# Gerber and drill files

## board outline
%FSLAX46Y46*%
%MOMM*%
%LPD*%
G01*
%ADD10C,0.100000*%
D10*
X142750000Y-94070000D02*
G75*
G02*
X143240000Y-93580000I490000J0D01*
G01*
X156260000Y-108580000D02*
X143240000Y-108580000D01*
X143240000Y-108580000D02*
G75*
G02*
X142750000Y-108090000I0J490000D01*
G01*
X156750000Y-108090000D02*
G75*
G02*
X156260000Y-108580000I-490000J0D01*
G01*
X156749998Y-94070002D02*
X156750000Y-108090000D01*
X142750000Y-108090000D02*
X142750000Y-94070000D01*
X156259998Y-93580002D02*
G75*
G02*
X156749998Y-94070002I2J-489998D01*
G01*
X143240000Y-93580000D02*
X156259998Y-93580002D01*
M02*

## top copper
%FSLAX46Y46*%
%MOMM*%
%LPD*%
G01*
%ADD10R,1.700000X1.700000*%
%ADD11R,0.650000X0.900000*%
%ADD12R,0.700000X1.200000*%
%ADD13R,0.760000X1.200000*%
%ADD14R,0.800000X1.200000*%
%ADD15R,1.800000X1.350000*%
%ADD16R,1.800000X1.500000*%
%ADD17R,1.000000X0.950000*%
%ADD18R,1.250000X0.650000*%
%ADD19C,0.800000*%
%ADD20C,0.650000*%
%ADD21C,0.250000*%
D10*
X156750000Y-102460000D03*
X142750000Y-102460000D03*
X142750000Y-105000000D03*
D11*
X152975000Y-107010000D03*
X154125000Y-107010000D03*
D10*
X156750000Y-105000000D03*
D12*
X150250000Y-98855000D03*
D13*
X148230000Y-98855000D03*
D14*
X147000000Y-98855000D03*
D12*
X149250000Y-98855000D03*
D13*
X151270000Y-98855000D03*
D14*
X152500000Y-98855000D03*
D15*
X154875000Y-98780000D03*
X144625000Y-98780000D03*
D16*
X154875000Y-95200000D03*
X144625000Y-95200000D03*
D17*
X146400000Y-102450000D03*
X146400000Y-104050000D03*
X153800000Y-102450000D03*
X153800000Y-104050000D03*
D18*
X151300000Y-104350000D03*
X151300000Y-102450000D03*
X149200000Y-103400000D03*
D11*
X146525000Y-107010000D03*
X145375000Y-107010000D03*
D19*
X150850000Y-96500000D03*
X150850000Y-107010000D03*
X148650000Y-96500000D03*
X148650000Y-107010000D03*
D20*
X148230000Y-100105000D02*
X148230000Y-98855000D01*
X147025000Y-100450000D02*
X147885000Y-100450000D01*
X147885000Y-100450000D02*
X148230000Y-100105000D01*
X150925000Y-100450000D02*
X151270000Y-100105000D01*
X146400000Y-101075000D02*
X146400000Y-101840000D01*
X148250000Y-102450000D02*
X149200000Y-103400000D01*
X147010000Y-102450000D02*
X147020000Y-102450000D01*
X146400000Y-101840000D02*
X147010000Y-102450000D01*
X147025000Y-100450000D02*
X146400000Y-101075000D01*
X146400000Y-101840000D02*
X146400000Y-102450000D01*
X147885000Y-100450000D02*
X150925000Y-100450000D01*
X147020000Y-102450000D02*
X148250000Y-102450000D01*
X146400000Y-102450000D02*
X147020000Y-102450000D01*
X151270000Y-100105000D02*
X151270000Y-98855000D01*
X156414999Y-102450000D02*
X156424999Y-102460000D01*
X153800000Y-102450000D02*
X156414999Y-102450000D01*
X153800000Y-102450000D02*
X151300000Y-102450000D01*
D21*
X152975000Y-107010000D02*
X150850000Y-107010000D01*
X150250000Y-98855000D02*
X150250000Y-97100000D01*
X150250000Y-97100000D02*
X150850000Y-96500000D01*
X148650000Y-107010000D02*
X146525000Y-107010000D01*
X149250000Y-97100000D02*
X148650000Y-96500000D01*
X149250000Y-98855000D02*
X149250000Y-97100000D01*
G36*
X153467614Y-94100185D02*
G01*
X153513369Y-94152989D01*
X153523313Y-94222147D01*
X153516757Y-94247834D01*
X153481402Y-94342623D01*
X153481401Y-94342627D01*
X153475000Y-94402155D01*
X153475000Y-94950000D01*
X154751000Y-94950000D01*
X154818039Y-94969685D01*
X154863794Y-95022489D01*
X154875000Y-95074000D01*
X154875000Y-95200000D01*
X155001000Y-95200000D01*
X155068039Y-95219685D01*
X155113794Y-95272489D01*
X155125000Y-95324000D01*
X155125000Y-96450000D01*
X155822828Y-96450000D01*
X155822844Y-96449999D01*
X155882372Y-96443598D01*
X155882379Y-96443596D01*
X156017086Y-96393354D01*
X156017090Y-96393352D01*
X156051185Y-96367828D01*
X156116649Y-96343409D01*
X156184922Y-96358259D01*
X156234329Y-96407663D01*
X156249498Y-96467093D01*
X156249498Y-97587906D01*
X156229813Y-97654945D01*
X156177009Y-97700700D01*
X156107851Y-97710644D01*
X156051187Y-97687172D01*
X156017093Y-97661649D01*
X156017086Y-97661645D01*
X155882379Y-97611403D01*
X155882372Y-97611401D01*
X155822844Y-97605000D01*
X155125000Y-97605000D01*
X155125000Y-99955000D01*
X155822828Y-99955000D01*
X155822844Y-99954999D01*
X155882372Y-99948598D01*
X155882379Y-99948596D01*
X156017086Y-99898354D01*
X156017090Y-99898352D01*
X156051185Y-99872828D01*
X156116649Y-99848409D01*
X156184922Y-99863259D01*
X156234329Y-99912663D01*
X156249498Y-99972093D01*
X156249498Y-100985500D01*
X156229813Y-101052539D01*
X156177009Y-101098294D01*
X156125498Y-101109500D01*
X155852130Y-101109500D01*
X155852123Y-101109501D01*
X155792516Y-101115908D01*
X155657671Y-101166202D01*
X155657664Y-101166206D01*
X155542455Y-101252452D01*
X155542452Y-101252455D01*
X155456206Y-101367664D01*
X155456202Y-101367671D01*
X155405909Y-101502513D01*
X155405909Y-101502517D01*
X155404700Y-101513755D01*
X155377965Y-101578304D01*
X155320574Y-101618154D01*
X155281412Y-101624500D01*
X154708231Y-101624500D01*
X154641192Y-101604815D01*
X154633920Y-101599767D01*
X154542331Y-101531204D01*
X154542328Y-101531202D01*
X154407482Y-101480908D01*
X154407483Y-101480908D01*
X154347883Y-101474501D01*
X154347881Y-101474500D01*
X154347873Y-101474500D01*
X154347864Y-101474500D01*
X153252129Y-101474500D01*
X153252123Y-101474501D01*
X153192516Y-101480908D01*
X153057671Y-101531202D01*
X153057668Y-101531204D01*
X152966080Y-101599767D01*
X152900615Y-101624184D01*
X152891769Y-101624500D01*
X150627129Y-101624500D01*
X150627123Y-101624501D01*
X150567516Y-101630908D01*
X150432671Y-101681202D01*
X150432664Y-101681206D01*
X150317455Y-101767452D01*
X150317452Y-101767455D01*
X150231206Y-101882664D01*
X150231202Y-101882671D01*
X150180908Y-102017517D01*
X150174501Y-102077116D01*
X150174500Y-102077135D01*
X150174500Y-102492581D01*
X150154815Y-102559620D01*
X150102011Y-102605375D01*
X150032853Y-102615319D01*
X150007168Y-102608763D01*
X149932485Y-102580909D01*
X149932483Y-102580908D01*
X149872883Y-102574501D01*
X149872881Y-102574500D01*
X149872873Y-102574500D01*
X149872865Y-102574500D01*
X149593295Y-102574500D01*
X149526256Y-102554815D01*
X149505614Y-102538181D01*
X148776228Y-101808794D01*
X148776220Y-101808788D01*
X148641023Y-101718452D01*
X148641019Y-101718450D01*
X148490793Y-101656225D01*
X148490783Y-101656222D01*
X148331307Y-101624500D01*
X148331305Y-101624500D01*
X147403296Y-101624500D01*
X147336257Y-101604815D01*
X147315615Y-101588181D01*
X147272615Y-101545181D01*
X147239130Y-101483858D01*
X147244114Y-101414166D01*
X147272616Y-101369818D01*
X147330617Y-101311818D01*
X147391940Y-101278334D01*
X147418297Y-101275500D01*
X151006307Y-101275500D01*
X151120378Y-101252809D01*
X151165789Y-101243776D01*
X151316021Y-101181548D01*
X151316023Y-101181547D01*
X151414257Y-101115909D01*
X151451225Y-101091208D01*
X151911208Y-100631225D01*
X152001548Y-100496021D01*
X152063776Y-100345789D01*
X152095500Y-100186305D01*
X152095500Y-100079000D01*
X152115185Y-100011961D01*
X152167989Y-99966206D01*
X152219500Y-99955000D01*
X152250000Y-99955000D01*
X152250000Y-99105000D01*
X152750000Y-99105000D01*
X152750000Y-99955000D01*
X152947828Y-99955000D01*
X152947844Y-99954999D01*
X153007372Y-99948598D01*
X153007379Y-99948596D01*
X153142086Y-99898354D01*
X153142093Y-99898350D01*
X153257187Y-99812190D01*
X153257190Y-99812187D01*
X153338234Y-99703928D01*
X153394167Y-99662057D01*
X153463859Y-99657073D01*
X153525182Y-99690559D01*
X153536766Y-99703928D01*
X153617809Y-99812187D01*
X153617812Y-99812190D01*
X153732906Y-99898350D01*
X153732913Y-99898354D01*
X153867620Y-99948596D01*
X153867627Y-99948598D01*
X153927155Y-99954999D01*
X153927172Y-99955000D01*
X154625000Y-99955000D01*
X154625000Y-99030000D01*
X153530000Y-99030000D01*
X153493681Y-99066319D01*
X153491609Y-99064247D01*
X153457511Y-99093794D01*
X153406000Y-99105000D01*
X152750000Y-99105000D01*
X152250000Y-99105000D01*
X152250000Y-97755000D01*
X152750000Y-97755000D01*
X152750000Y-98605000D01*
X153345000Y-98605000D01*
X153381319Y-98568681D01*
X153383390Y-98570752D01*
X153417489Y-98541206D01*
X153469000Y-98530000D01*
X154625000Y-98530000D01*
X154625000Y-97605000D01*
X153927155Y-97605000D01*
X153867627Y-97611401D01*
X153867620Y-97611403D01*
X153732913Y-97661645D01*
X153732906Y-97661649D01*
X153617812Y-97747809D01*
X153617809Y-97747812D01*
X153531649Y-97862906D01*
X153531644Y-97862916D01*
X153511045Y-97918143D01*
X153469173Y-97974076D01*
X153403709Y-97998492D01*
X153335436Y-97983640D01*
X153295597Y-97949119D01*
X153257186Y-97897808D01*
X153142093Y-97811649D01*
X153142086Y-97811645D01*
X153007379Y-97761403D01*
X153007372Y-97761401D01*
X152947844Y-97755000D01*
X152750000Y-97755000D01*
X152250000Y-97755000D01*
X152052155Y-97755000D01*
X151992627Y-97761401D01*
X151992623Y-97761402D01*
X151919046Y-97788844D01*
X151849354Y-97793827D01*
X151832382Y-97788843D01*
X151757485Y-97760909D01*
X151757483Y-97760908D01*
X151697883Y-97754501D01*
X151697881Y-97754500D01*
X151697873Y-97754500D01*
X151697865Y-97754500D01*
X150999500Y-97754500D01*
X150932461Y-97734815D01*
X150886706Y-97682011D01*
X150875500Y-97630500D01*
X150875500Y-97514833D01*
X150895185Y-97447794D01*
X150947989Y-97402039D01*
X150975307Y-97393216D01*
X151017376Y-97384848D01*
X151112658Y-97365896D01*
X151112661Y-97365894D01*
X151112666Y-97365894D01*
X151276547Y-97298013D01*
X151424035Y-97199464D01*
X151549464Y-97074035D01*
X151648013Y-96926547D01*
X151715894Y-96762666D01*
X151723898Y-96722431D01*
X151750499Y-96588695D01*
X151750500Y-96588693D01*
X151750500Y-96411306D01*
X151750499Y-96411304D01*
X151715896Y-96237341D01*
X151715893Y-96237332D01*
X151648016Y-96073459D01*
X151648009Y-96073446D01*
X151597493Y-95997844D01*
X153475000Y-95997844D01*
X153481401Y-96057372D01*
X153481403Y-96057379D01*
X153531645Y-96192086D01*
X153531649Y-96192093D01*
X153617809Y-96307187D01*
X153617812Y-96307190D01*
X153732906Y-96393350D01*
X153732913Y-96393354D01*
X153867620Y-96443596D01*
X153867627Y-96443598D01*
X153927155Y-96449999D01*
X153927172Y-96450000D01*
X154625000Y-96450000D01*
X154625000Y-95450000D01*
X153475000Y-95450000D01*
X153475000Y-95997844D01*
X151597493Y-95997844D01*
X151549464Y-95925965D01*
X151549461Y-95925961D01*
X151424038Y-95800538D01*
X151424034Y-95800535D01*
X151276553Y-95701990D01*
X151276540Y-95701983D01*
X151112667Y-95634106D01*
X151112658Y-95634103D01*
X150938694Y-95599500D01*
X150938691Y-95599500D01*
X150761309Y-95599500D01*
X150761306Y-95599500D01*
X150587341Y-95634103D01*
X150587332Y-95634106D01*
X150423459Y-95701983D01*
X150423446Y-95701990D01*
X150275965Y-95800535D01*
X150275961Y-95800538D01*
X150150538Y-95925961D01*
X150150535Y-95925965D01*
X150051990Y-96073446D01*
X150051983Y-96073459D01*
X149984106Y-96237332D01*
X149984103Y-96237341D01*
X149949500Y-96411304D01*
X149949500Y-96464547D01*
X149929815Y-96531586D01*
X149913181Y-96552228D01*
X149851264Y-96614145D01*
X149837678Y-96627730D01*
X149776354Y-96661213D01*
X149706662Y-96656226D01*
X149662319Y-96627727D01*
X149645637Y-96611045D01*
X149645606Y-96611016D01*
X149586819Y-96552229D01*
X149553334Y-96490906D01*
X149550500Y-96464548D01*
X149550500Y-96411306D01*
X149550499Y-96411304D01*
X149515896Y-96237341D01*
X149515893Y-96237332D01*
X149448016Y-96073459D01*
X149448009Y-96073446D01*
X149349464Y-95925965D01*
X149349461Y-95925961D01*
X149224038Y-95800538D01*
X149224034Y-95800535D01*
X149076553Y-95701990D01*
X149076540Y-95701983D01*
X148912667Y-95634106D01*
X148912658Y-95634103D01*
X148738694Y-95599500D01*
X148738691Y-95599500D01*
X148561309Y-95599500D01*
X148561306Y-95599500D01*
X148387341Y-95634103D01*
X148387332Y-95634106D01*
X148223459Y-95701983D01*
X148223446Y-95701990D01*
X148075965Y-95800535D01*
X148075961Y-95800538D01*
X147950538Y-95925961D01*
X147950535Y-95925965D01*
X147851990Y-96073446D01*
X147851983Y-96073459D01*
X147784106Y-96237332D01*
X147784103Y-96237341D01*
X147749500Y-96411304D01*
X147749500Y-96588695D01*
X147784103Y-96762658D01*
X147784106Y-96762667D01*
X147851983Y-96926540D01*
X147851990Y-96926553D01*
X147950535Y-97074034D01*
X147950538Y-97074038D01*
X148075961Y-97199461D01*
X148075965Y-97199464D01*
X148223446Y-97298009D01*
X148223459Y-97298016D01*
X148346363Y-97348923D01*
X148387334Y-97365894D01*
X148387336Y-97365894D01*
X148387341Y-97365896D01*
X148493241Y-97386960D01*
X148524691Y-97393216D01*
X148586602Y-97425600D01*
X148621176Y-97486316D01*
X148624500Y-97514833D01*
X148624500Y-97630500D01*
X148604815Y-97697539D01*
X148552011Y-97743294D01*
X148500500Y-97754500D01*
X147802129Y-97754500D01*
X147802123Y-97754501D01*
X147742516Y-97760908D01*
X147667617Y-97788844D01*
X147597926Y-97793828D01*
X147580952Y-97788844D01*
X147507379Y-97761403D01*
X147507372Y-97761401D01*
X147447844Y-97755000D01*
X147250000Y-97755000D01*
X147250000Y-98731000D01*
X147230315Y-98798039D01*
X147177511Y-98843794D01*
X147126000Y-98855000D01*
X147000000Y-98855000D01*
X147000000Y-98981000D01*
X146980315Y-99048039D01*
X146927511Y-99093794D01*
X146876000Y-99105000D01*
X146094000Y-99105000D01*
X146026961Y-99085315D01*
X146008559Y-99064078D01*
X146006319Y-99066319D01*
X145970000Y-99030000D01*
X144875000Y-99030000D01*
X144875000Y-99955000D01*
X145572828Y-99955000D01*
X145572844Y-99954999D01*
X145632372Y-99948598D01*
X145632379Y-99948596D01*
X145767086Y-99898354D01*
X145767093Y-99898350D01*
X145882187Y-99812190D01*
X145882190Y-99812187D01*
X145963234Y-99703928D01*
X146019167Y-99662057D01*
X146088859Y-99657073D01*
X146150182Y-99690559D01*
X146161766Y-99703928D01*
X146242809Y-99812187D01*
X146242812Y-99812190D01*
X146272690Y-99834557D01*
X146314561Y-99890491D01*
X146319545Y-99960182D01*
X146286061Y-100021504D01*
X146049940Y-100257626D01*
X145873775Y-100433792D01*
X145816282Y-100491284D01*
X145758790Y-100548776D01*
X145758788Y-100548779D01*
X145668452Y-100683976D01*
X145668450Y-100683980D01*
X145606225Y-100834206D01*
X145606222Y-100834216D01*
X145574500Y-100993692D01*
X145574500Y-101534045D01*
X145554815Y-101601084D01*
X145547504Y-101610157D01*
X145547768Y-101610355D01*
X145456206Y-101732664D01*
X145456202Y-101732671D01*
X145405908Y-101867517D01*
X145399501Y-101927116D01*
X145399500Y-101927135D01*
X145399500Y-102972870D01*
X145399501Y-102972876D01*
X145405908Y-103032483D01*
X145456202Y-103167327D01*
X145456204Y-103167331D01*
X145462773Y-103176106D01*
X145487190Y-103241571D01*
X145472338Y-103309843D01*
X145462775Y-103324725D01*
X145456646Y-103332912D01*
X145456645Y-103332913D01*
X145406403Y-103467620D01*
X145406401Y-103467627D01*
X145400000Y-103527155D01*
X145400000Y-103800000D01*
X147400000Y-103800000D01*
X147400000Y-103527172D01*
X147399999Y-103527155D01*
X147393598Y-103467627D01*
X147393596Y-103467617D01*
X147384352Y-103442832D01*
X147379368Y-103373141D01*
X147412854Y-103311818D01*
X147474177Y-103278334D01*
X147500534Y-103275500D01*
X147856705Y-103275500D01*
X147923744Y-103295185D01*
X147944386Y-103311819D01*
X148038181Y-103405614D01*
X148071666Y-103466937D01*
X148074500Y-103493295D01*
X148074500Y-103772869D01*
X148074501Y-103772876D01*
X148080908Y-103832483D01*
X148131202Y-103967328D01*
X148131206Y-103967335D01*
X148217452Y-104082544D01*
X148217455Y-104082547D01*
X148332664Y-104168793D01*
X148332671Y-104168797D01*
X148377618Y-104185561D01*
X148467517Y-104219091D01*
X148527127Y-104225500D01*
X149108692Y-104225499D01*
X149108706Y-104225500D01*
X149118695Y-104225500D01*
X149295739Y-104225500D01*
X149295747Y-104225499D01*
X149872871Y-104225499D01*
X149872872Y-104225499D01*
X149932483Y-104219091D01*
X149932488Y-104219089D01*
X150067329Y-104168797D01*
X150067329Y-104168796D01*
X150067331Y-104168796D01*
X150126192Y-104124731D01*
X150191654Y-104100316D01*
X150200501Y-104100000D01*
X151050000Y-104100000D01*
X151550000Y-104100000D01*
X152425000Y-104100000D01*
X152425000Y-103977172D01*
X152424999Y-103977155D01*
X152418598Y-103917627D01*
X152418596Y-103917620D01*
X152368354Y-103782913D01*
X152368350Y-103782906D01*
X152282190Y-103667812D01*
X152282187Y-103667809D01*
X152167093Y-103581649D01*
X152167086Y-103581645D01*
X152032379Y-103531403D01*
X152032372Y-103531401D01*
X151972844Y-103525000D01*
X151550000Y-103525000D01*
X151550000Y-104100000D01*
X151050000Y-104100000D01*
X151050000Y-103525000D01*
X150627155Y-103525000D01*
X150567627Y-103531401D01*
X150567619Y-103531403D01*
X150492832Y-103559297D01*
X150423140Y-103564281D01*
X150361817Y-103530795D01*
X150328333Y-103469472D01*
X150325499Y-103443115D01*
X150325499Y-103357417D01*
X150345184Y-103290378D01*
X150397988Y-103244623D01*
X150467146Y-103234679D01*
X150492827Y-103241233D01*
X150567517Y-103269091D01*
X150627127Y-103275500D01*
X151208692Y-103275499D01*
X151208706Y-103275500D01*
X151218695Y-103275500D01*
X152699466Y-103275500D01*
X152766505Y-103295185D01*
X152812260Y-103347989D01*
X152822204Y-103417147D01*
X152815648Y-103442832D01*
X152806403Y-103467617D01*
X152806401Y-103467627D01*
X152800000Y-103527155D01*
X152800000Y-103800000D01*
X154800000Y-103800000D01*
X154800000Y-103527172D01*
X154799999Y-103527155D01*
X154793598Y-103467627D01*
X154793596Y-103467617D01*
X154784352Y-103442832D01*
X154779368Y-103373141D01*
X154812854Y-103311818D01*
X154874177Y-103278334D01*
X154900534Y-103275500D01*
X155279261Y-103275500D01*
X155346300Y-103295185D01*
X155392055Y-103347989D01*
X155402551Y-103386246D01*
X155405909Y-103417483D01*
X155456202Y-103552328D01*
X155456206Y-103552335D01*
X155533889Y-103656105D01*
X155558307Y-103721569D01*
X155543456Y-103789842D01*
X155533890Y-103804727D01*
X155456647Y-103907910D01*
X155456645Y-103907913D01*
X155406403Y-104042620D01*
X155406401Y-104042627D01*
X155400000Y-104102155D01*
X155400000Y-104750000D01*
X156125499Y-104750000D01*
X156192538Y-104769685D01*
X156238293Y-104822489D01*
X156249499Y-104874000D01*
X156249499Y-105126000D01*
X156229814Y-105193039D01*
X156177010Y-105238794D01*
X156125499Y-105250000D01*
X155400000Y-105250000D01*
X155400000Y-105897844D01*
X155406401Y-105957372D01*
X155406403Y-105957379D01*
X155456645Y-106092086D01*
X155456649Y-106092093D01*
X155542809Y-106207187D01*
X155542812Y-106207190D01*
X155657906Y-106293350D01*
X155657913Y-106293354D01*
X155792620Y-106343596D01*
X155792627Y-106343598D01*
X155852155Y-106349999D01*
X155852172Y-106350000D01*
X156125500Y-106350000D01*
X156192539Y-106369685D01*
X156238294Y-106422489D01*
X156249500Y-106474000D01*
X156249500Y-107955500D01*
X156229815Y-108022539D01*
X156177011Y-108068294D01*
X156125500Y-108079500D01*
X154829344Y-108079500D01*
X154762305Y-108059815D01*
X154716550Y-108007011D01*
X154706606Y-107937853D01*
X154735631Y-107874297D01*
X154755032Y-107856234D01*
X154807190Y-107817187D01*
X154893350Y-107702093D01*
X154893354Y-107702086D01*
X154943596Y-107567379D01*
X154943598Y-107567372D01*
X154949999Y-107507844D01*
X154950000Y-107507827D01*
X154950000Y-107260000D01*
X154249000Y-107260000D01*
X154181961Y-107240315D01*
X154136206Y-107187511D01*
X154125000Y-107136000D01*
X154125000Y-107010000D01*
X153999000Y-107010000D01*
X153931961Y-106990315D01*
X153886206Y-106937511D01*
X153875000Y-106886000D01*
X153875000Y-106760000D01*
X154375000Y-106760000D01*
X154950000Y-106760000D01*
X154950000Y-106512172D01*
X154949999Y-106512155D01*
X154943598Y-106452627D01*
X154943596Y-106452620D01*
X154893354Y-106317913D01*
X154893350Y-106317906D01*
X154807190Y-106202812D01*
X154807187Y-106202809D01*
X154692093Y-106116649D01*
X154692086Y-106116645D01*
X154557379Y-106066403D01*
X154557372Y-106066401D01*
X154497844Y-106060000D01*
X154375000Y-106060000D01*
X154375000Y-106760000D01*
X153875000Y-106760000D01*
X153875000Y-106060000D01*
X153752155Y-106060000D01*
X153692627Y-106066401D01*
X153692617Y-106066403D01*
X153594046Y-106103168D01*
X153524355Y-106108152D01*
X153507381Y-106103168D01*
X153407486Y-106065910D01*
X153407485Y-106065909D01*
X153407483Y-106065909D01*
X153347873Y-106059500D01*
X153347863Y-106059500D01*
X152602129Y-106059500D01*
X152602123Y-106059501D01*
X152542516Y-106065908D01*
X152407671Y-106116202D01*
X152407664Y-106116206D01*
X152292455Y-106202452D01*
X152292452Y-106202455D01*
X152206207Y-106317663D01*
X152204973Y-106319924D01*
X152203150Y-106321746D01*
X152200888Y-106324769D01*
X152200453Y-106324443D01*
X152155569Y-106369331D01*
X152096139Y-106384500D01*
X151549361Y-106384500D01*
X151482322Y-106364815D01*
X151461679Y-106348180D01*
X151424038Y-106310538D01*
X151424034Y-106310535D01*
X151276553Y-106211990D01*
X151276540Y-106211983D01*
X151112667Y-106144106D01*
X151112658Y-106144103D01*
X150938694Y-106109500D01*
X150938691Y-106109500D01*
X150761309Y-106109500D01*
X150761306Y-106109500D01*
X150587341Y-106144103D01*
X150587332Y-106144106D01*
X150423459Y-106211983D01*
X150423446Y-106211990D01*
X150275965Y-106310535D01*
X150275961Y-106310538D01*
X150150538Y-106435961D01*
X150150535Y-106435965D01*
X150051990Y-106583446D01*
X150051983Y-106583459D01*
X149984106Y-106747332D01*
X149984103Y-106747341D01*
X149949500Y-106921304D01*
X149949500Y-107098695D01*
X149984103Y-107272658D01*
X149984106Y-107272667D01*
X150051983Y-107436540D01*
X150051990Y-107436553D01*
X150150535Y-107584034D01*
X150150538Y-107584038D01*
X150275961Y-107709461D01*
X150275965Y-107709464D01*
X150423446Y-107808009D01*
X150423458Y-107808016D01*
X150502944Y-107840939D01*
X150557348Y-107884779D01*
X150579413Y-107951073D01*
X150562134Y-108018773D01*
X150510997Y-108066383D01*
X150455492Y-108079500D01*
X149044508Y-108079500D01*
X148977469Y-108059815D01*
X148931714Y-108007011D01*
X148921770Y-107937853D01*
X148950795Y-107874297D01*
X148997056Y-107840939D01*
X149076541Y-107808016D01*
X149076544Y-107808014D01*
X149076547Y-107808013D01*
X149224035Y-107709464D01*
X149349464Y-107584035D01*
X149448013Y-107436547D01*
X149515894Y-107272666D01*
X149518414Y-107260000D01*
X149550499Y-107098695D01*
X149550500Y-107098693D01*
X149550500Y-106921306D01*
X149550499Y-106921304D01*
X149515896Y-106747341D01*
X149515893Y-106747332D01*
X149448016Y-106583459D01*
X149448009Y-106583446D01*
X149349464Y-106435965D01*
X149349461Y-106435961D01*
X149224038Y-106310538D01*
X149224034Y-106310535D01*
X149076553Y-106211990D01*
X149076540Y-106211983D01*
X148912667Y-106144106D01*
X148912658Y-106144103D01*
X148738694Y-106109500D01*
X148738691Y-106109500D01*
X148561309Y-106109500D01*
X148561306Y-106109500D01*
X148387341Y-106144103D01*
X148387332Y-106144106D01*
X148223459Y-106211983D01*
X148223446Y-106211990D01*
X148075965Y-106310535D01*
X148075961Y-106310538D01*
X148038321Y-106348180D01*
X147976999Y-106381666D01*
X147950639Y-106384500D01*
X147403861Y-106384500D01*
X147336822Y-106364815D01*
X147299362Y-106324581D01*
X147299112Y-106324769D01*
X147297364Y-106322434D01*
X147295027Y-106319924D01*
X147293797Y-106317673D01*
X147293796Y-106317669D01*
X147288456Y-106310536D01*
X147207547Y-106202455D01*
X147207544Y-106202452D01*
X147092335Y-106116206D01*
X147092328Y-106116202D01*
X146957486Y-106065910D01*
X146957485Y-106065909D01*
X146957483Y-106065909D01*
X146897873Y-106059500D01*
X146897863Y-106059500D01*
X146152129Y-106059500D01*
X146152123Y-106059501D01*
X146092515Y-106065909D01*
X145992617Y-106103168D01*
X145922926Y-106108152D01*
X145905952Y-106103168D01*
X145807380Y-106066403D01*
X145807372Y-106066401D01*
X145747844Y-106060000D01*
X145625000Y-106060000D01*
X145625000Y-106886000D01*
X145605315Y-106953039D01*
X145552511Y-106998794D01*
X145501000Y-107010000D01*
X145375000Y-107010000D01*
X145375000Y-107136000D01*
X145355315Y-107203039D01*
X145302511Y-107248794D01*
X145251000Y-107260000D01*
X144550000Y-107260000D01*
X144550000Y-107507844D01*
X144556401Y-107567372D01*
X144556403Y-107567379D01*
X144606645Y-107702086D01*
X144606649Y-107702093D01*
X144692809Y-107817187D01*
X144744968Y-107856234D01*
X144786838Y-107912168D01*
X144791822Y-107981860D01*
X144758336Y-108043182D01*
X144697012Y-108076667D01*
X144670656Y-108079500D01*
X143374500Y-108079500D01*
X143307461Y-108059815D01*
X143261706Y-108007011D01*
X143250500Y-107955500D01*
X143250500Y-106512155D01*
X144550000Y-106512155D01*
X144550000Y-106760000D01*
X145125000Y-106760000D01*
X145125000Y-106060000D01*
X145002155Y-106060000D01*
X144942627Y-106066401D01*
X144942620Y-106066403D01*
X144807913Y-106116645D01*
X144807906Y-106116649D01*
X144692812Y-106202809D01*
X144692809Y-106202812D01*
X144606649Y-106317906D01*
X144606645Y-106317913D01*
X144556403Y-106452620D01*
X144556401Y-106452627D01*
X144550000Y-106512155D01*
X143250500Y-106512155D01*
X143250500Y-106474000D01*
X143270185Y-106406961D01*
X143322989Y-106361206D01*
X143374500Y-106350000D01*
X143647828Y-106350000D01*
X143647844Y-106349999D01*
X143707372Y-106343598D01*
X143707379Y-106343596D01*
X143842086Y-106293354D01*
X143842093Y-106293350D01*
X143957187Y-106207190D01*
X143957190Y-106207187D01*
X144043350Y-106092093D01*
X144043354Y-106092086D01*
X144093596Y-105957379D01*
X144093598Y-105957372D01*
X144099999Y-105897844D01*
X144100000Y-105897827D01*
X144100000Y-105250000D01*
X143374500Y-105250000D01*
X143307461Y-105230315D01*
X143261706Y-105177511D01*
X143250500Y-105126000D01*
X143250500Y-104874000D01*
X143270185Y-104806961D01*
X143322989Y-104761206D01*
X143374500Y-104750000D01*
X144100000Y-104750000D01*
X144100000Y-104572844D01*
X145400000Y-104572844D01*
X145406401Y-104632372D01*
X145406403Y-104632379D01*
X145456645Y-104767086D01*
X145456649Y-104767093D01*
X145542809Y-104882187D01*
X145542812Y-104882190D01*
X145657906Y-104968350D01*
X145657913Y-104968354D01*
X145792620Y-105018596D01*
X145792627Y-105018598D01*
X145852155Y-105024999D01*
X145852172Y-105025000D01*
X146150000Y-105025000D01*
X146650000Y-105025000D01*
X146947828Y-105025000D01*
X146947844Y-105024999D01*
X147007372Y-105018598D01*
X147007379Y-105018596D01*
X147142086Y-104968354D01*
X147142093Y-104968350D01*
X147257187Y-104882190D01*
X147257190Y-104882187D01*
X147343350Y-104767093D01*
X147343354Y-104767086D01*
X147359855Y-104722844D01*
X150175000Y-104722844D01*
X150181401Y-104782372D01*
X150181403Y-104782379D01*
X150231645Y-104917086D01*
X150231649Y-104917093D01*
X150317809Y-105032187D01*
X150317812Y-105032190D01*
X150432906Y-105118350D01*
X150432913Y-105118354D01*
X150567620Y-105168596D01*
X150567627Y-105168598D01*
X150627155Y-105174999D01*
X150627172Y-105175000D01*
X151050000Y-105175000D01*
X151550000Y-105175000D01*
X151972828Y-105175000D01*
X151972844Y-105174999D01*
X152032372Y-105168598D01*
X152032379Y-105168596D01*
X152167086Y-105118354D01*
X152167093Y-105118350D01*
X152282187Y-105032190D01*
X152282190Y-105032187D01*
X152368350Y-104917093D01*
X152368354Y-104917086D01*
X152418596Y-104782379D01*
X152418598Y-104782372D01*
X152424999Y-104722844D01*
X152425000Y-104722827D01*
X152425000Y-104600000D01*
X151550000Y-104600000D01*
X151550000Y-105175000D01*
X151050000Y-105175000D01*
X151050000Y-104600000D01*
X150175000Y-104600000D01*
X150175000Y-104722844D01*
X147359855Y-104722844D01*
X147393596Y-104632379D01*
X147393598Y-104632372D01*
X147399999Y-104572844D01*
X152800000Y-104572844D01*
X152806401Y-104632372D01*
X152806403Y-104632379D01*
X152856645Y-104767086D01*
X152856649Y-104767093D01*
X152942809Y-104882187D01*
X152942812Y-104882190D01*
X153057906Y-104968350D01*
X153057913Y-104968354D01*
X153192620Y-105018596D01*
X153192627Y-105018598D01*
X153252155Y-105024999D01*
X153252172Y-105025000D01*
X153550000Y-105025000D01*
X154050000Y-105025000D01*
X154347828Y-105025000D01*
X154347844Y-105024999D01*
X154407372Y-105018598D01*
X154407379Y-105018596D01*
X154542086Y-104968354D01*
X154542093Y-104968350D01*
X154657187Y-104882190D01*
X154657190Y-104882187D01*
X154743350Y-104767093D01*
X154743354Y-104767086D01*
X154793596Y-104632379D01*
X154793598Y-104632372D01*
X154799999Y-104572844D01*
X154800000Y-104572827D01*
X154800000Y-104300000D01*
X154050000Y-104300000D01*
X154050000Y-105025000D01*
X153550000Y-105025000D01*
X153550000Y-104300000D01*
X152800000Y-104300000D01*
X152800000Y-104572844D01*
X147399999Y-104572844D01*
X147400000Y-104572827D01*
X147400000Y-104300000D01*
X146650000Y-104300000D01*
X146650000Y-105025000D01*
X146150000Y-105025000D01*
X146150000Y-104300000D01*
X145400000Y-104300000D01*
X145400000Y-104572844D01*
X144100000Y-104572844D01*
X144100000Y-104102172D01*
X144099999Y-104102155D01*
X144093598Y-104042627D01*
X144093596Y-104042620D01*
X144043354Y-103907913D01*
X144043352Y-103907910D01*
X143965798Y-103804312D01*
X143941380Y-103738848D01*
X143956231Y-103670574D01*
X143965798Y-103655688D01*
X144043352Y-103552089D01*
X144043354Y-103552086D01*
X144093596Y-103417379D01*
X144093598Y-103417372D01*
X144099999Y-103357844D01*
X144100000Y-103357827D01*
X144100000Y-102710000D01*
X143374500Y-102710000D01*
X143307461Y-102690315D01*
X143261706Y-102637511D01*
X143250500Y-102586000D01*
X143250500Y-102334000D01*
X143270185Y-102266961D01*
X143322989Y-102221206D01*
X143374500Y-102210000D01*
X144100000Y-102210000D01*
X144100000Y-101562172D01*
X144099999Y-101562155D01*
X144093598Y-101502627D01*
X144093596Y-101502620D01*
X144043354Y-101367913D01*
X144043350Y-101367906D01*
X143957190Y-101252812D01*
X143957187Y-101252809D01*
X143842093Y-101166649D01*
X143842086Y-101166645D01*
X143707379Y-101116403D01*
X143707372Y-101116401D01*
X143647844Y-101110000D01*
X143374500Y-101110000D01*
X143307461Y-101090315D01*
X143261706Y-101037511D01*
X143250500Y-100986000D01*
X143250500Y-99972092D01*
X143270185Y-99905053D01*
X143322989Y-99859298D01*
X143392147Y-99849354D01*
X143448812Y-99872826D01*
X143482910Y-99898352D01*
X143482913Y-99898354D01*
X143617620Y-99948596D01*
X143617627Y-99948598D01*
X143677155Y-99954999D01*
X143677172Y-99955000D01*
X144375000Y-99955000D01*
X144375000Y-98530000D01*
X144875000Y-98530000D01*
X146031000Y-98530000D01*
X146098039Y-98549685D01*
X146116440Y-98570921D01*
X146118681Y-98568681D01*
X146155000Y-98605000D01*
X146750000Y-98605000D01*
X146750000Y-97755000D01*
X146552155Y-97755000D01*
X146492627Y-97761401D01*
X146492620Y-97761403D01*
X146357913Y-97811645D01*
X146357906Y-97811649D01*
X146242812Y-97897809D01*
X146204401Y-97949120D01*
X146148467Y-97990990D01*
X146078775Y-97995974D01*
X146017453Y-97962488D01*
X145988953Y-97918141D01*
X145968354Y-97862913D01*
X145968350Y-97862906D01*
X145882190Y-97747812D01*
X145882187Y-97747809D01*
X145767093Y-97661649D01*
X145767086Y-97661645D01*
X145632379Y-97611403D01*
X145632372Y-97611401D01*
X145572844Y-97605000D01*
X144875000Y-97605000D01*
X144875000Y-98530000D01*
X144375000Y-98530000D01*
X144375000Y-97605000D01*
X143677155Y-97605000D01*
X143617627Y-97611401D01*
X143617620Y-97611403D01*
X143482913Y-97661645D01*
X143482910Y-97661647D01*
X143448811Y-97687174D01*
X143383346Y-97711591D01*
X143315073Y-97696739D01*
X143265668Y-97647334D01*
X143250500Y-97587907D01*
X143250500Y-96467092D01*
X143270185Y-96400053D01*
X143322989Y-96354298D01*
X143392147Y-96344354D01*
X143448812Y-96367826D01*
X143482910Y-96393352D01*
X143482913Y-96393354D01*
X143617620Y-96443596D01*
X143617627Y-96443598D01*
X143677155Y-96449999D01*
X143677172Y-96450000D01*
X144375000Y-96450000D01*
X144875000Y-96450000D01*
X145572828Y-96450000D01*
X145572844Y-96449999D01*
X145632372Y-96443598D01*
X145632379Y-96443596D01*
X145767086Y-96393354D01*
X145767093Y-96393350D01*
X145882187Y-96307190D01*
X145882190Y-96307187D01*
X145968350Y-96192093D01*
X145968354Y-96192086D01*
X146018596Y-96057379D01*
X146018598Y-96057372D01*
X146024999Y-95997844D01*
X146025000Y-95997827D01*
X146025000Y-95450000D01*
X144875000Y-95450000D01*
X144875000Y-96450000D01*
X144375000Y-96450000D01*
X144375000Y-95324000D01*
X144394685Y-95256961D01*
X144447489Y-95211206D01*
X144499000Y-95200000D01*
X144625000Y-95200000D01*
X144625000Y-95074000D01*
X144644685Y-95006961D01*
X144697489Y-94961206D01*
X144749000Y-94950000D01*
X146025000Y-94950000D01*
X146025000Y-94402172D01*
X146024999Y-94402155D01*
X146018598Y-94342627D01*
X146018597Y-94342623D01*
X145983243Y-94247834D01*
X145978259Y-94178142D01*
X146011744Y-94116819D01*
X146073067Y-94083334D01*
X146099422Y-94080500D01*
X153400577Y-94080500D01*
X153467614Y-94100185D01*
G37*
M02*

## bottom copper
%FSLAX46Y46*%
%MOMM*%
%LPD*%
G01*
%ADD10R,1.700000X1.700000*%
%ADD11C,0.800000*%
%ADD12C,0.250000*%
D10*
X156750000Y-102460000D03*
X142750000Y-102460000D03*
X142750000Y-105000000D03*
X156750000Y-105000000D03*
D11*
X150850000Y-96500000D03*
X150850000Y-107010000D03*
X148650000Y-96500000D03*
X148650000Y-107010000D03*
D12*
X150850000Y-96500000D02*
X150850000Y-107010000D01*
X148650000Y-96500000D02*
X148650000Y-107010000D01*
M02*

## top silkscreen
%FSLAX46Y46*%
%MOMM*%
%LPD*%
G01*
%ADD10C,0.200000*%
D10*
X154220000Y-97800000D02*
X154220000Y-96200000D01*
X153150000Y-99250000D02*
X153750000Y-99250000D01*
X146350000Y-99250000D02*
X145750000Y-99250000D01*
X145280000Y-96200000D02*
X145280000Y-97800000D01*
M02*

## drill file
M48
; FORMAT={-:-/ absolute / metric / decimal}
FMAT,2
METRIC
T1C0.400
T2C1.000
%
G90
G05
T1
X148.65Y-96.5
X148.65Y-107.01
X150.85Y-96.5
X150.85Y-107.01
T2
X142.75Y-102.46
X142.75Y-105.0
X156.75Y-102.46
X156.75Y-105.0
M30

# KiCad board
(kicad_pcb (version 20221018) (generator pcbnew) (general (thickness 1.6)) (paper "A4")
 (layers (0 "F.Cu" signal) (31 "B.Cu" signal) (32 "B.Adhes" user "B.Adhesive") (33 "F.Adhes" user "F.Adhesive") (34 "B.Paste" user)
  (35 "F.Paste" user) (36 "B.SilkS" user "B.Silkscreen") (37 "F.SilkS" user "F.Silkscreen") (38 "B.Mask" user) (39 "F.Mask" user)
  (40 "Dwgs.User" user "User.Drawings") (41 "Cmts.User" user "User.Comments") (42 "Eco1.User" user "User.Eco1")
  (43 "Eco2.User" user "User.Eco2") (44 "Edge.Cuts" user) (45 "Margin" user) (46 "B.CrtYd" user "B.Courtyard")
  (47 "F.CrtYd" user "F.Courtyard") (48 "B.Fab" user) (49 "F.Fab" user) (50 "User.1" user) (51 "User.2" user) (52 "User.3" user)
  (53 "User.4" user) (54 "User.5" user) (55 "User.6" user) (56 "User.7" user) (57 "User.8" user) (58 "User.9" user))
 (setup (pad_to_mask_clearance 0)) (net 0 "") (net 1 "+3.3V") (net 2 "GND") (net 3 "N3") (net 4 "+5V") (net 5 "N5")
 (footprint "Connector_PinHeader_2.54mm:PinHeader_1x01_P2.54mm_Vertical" (layer "F.Cu") (at 156.75 102.46 180)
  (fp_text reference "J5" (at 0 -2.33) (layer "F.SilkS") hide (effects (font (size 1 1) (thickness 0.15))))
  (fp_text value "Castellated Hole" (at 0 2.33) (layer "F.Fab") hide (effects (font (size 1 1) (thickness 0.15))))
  (pad "1" thru_hole rect (at 0 0 180) (size 1.7 1.7) (drill 1) (layers "*.Cu" "*.Mask") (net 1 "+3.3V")))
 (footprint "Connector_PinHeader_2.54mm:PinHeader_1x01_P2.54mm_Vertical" (layer "F.Cu") (at 142.75 102.46 90)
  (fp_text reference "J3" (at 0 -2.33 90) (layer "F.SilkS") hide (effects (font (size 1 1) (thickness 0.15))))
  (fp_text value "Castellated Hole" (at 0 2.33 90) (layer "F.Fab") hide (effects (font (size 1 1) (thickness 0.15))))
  (pad "1" thru_hole rect (at 0 0 90) (size 1.7 1.7) (drill 1) (layers "*.Cu" "*.Mask") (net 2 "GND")))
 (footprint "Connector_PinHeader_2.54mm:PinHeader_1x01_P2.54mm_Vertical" (layer "F.Cu") (at 142.75 105)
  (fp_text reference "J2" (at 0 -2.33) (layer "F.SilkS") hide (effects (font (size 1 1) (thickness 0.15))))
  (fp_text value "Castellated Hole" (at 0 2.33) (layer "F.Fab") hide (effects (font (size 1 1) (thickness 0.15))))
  (pad "1" thru_hole rect (at 0 0) (size 1.7 1.7) (drill 1) (layers "*.Cu" "*.Mask") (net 2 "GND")))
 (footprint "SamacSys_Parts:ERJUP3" (layer "F.Cu") (at 153.55 107.01)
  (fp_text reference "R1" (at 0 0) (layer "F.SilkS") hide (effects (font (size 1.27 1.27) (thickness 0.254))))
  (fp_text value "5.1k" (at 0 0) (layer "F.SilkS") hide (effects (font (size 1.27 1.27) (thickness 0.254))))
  (pad "1" smd rect (at -0.575 0) (size 0.65 0.9) (layers "F.Cu" "F.Paste" "F.Mask") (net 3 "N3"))
  (pad "2" smd rect (at 0.575 0) (size 0.65 0.9) (layers "F.Cu" "F.Paste" "F.Mask") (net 2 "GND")))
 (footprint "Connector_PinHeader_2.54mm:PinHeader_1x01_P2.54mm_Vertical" (layer "F.Cu") (at 156.75 105 180)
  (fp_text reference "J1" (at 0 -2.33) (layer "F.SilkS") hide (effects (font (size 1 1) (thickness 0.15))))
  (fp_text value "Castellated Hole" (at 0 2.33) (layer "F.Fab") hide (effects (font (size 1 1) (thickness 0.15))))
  (pad "1" thru_hole rect (at 0 0 180) (size 1.7 1.7) (drill 1) (layers "*.Cu" "*.Mask") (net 2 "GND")))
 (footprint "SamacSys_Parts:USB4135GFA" (layer "F.Cu") (at 149.75 95.8 180)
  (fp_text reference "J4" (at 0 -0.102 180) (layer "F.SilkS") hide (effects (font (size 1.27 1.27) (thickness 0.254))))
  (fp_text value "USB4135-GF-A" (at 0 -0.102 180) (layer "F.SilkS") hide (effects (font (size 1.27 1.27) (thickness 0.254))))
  (fp_line (start -4.47 -2) (end -4.47 -0.4) (stroke (width 0.2) (type solid)) (layer "F.SilkS"))
  (fp_line (start -3.4 -3.45) (end -4 -3.45) (stroke (width 0.2) (type solid)) (layer "F.SilkS"))
  (fp_line (start 3.4 -3.45) (end 4 -3.45) (stroke (width 0.2) (type solid)) (layer "F.SilkS"))
  (fp_line (start 4.47 -0.4) (end 4.47 -2) (stroke (width 0.2) (type solid)) (layer "F.SilkS"))
  (pad "A5" smd rect (at -0.5 -3.055 180) (size 0.7 1.2) (layers "F.Cu" "F.Paste" "F.Mask") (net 3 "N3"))
  (pad "A9" smd rect (at 1.52 -3.055 180) (size 0.76 1.2) (layers "F.Cu" "F.Paste" "F.Mask") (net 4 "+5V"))
  (pad "A12" smd rect (at 2.75 -3.055 180) (size 0.8 1.2) (layers "F.Cu" "F.Paste" "F.Mask") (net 2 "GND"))
  (pad "B5" smd rect (at 0.5 -3.055 180) (size 0.7 1.2) (layers "F.Cu" "F.Paste" "F.Mask") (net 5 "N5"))
  (pad "B9" smd rect (at -1.52 -3.055 180) (size 0.76 1.2) (layers "F.Cu" "F.Paste" "F.Mask") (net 4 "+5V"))
  (pad "B12" smd rect (at -2.75 -3.055 180) (size 0.8 1.2) (layers "F.Cu" "F.Paste" "F.Mask") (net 2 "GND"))
  (pad "MP1" smd rect (at -5.125 -2.98 270) (size 1.35 1.8) (layers "F.Cu" "F.Paste" "F.Mask") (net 2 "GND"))
  (pad "MP2" smd rect (at 5.125 -2.98 270) (size 1.35 1.8) (layers "F.Cu" "F.Paste" "F.Mask") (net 2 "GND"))
  (pad "MP3" smd rect (at -5.125 0.6 270) (size 1.5 1.8) (layers "F.Cu" "F.Paste" "F.Mask") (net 2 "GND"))
  (pad "MP4" smd rect (at 5.125 0.6 270) (size 1.5 1.8) (layers "F.Cu" "F.Paste" "F.Mask") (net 2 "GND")))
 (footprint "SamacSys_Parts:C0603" (layer "F.Cu") (at 146.4 103.25 -90)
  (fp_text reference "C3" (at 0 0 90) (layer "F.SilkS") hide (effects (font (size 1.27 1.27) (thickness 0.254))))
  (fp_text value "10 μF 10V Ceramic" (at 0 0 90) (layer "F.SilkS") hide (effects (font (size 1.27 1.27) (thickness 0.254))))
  (pad "1" smd rect (at -0.8 0 270) (size 0.95 1) (layers "F.Cu" "F.Paste" "F.Mask") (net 4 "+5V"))
  (pad "2" smd rect (at 0.8 0 270) (size 0.95 1) (layers "F.Cu" "F.Paste" "F.Mask") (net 2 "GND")))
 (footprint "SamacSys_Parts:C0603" (layer "F.Cu") (at 153.8 103.25 -90)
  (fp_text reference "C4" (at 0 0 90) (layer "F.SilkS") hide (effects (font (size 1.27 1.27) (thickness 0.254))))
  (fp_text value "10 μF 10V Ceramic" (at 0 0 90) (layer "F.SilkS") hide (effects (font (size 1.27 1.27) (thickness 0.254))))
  (pad "1" smd rect (at -0.8 0 270) (size 0.95 1) (layers "F.Cu" "F.Paste" "F.Mask") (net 1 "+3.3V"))
  (pad "2" smd rect (at 0.8 0 270) (size 0.95 1) (layers "F.Cu" "F.Paste" "F.Mask") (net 2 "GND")))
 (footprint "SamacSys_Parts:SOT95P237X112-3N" (layer "F.Cu") (at 150.25 103.4 180)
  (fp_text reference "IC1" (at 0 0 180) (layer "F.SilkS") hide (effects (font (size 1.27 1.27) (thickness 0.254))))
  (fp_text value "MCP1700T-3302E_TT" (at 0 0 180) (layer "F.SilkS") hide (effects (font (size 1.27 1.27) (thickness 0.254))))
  (pad "1" smd rect (at -1.05 -0.95 270) (size 0.65 1.25) (layers "F.Cu" "F.Paste" "F.Mask") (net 2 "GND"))
  (pad "2" smd rect (at -1.05 0.95 270) (size 0.65 1.25) (layers "F.Cu" "F.Paste" "F.Mask") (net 1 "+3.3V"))
  (pad "3" smd rect (at 1.05 0 270) (size 0.65 1.25) (layers "F.Cu" "F.Paste" "F.Mask") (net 4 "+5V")))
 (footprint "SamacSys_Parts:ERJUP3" (layer "F.Cu") (at 145.95 107.01 180)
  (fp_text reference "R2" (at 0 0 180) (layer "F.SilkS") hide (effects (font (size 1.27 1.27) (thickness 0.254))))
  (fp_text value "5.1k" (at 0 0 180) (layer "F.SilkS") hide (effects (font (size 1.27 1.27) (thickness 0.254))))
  (pad "1" smd rect (at -0.575 0 180) (size 0.65 0.9) (layers "F.Cu" "F.Paste" "F.Mask") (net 5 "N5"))
  (pad "2" smd rect (at 0.575 0 180) (size 0.65 0.9) (layers "F.Cu" "F.Paste" "F.Mask") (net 2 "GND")))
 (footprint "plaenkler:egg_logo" (layer "B.Cu") (at 153.725 97.025 180)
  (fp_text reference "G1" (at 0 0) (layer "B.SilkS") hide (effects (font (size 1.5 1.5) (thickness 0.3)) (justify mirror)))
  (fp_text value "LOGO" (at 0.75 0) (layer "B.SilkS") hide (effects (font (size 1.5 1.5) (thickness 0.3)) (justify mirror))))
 (gr_arc (start 142.75 94.07) (mid 142.893518 93.723518) (end 143.24 93.58) (stroke (width 0.1) (type default)) (layer "Edge.Cuts"))
 (gr_line (start 156.26 108.58) (end 143.24 108.58) (stroke (width 0.1) (type default)) (layer "Edge.Cuts"))
 (gr_arc (start 143.24 108.58) (mid 142.893518 108.436482) (end 142.75 108.09) (stroke (width 0.1) (type default)) (layer "Edge.Cuts"))
 (gr_arc (start 156.75 108.09) (mid 156.606482 108.436482) (end 156.26 108.58) (stroke (width 0.1) (type default)) (layer "Edge.Cuts"))
 (gr_line (start 156.749998 94.070002) (end 156.75 108.09) (stroke (width 0.1) (type default)) (layer "Edge.Cuts"))
 (gr_line (start 142.75 108.09) (end 142.75 94.07) (stroke (width 0.1) (type default)) (layer "Edge.Cuts"))
 (gr_arc (start 156.259998 93.580002) (mid 156.606481 93.723519) (end 156.749998 94.070002) (stroke (width 0.1) (type default))
  (layer "Edge.Cuts"))
 (gr_line (start 143.24 93.58) (end 156.259998 93.580002) (stroke (width 0.1) (type default)) (layer "Edge.Cuts"))
 (segment (start 148.23 100.105) (end 148.23 98.855) (width 0.65) (layer "F.Cu") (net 4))
 (segment (start 147.025 100.45) (end 147.885 100.45) (width 0.65) (layer "F.Cu") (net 4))
 (segment (start 147.885 100.45) (end 148.23 100.105) (width 0.65) (layer "F.Cu") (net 4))
 (segment (start 150.925 100.45) (end 151.27 100.105) (width 0.65) (layer "F.Cu") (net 4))
 (segment (start 146.4 101.075) (end 146.4 101.84) (width 0.65) (layer "F.Cu") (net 4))
 (segment (start 148.25 102.45) (end 149.2 103.4) (width 0.65) (layer "F.Cu") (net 4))
 (segment (start 147.01 102.45) (end 147.02 102.45) (width 0.65) (layer "F.Cu") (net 4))
 (segment (start 146.4 101.84) (end 147.01 102.45) (width 0.65) (layer "F.Cu") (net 4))
 (segment (start 147.025 100.45) (end 146.4 101.075) (width 0.65) (layer "F.Cu") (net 4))
 (segment (start 146.4 101.84) (end 146.4 102.45) (width 0.65) (layer "F.Cu") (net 4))
 (segment (start 147.885 100.45) (end 150.925 100.45) (width 0.65) (layer "F.Cu") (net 4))
 (segment (start 147.02 102.45) (end 148.25 102.45) (width 0.65) (layer "F.Cu") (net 4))
 (segment (start 146.4 102.45) (end 147.02 102.45) (width 0.65) (layer "F.Cu") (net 4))
 (segment (start 151.27 100.105) (end 151.27 98.855) (width 0.65) (layer "F.Cu") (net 4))
 (segment (start 156.414999 102.45) (end 156.424999 102.46) (width 0.65) (layer "F.Cu") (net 1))
 (segment (start 153.8 102.45) (end 156.414999 102.45) (width 0.65) (layer "F.Cu") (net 1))
 (segment (start 153.8 102.45) (end 151.3 102.45) (width 0.65) (layer "F.Cu") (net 1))
 (segment (start 152.975 107.01) (end 150.85 107.01) (width 0.25) (layer "F.Cu") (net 3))
 (segment (start 150.25 98.855) (end 150.25 97.1) (width 0.25) (layer "F.Cu") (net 3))
 (segment (start 150.25 97.1) (end 150.85 96.5) (width 0.25) (layer "F.Cu") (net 3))
 (via (at 150.85 96.5) (size 0.8) (drill 0.4) (layers "F.Cu" "B.Cu") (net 3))
 (via (at 150.85 107.01) (size 0.8) (drill 0.4) (layers "F.Cu" "B.Cu") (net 3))
 (segment (start 150.85 96.5) (end 150.85 107.01) (width 0.25) (layer "B.Cu") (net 3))
 (segment (start 148.65 107.01) (end 146.525 107.01) (width 0.25) (layer "F.Cu") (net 5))
 (segment (start 149.25 97.1) (end 148.65 96.5) (width 0.25) (layer "F.Cu") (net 5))
 (segment (start 149.25 98.855) (end 149.25 97.1) (width 0.25) (layer "F.Cu") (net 5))
 (via (at 148.65 96.5) (size 0.8) (drill 0.4) (layers "F.Cu" "B.Cu") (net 5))
 (via (at 148.65 107.01) (size 0.8) (drill 0.4) (layers "F.Cu" "B.Cu") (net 5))
 (segment (start 148.65 96.5) (end 148.65 107.01) (width 0.25) (layer "B.Cu") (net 5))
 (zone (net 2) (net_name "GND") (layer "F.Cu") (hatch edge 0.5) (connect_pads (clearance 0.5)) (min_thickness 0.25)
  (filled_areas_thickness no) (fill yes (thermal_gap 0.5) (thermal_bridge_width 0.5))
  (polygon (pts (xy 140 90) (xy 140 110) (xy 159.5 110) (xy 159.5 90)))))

